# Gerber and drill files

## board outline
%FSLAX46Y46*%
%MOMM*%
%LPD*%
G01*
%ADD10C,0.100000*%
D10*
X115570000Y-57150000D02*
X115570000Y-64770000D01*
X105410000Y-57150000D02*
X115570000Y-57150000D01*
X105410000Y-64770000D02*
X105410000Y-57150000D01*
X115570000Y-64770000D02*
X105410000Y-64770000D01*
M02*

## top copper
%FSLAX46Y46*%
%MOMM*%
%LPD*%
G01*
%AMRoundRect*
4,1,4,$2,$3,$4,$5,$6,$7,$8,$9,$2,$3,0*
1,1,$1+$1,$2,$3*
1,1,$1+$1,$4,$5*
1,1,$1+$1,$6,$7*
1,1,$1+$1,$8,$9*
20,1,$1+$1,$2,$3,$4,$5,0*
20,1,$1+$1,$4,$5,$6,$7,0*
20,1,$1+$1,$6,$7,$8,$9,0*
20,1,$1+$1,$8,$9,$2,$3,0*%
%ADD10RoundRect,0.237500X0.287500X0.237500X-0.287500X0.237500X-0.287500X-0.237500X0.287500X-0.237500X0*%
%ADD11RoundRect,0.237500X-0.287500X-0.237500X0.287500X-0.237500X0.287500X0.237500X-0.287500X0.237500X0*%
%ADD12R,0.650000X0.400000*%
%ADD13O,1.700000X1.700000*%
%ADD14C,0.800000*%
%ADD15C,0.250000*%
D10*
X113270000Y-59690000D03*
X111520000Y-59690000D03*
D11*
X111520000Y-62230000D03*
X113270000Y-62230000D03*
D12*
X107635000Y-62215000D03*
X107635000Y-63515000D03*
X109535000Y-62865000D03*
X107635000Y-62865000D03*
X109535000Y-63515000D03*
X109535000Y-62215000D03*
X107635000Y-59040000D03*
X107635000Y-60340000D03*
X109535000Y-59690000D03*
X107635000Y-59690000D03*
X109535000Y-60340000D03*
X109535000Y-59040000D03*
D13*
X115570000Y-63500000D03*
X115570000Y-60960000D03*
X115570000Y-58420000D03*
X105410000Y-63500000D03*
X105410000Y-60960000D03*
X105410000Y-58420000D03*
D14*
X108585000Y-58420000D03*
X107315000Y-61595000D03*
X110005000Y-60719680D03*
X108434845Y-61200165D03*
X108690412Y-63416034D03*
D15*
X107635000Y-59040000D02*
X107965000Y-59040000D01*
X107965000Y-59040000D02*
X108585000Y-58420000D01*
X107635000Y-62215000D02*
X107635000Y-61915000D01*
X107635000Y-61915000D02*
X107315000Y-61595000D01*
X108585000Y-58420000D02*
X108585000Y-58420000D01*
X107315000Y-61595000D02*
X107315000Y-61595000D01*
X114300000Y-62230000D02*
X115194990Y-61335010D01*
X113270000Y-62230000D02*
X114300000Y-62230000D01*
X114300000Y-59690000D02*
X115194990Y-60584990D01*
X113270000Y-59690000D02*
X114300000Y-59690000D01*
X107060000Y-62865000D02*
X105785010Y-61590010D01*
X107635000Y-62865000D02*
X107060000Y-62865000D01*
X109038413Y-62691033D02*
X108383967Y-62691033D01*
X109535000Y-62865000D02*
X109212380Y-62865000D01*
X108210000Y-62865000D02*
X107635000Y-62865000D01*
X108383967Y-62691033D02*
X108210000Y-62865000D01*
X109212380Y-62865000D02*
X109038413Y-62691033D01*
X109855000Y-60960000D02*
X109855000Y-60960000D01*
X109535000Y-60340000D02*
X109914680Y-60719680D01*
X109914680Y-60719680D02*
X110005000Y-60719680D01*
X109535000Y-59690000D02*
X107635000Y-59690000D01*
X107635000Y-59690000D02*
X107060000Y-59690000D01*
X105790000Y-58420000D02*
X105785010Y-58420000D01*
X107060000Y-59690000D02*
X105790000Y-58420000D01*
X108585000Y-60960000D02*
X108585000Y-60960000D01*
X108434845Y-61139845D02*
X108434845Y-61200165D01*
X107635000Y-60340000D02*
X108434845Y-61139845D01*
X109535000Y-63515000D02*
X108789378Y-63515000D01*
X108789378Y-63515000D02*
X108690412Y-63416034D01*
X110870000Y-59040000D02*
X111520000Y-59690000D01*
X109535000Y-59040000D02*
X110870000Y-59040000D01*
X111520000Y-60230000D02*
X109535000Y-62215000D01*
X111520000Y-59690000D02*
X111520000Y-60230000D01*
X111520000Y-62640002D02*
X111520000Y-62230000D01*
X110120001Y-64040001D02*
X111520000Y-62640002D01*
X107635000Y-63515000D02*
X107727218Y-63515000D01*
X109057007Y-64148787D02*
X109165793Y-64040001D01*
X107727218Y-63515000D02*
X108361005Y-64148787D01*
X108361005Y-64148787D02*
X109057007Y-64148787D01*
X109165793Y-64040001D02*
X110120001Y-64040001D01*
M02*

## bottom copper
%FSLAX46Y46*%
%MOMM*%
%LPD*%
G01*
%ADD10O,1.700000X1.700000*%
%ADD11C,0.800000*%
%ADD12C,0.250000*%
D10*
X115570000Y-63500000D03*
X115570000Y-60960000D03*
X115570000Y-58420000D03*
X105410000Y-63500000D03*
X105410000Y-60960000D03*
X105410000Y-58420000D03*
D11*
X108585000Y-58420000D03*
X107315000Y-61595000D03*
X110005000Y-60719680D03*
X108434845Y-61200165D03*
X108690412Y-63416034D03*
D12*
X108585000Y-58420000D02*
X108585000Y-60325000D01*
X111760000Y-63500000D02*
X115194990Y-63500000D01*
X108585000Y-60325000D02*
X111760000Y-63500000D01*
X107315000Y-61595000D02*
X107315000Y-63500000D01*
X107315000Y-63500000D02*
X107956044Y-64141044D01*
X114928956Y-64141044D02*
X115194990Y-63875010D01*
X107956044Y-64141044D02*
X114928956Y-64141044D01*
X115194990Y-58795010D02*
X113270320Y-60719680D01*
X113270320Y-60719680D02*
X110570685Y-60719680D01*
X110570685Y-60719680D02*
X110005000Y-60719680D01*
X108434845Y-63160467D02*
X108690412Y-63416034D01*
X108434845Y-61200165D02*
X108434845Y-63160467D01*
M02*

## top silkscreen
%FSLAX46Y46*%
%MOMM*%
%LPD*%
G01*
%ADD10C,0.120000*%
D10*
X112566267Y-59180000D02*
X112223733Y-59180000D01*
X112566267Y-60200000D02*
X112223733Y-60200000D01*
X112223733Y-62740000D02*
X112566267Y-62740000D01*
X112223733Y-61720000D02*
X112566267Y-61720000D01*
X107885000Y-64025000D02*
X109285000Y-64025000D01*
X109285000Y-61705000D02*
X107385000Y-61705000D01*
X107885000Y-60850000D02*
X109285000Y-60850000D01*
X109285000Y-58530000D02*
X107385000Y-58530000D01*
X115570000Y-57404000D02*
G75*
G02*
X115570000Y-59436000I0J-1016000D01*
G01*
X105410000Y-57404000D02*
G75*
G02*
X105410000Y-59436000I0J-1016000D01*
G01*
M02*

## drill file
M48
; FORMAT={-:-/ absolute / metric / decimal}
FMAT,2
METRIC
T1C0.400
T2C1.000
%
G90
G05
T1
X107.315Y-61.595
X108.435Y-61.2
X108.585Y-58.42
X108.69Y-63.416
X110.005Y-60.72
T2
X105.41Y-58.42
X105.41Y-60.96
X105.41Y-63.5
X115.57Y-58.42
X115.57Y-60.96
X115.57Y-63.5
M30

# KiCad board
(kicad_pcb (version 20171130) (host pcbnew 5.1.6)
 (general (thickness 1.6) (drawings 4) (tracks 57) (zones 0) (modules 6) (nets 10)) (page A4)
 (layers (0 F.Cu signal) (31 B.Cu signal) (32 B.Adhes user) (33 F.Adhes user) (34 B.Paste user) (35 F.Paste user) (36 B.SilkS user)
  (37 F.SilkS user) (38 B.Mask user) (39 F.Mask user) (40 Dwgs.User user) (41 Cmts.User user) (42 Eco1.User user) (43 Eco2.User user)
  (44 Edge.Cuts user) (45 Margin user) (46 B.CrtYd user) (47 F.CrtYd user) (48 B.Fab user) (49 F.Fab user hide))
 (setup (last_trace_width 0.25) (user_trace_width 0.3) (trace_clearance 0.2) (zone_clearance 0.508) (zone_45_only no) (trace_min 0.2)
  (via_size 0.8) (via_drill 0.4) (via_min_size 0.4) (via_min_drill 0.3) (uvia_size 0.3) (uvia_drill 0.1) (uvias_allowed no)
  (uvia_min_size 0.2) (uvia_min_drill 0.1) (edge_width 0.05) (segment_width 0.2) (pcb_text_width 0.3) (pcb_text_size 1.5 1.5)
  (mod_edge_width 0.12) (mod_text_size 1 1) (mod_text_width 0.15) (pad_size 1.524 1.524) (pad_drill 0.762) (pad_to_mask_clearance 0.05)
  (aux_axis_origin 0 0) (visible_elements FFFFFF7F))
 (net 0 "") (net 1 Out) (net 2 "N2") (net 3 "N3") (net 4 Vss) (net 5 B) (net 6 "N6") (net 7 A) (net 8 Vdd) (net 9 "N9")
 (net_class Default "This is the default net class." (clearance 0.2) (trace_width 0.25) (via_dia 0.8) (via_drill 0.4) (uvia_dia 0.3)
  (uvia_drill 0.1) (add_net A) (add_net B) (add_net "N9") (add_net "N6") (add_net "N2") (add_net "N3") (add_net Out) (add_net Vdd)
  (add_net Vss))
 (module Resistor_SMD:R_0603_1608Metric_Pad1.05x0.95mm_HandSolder (layer F.Cu) (at 112.395 59.69 180)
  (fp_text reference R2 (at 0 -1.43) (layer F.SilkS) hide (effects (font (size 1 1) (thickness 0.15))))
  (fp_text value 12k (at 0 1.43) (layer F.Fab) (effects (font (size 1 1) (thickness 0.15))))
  (fp_line (start -0.171267 0.51) (end 0.171267 0.51) (layer F.SilkS) (width 0.12))
  (fp_line (start -0.171267 -0.51) (end 0.171267 -0.51) (layer F.SilkS) (width 0.12))
  (pad 1 smd roundrect (at -0.875 0 180) (size 1.05 0.95) (layers F.Cu F.Paste F.Mask) (roundrect_rratio 0.25) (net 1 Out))
  (pad 2 smd roundrect (at 0.875 0 180) (size 1.05 0.95) (layers F.Cu F.Paste F.Mask) (roundrect_rratio 0.25) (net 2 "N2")))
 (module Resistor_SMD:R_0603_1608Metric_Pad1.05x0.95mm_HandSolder (layer F.Cu) (at 112.395 62.23)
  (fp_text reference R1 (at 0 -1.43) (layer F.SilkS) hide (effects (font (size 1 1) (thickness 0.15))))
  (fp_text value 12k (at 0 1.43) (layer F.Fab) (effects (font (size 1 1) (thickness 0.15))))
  (fp_line (start -0.171267 0.51) (end 0.171267 0.51) (layer F.SilkS) (width 0.12))
  (fp_line (start -0.171267 -0.51) (end 0.171267 -0.51) (layer F.SilkS) (width 0.12))
  (pad 1 smd roundrect (at -0.875 0) (size 1.05 0.95) (layers F.Cu F.Paste F.Mask) (roundrect_rratio 0.25) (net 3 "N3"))
  (pad 2 smd roundrect (at 0.875 0) (size 1.05 0.95) (layers F.Cu F.Paste F.Mask) (roundrect_rratio 0.25) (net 1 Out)))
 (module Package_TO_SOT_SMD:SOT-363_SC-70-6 (layer F.Cu) (at 108.585 62.865)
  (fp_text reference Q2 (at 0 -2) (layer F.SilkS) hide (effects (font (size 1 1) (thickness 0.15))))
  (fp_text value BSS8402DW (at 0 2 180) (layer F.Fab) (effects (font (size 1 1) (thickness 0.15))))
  (fp_line (start -0.7 1.16) (end 0.7 1.16) (layer F.SilkS) (width 0.12))
  (fp_line (start 0.7 -1.16) (end -1.2 -1.16) (layer F.SilkS) (width 0.12))
  (pad 1 smd rect (at -0.95 -0.65) (size 0.65 0.4) (layers F.Cu F.Paste F.Mask) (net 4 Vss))
  (pad 3 smd rect (at -0.95 0.65) (size 0.65 0.4) (layers F.Cu F.Paste F.Mask) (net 3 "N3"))
  (pad 5 smd rect (at 0.95 0) (size 0.65 0.4) (layers F.Cu F.Paste F.Mask) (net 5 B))
  (pad 2 smd rect (at -0.95 0) (size 0.65 0.4) (layers F.Cu F.Paste F.Mask) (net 5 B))
  (pad 4 smd rect (at 0.95 0.65) (size 0.65 0.4) (layers F.Cu F.Paste F.Mask) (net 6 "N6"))
  (pad 6 smd rect (at 0.95 -0.65) (size 0.65 0.4) (layers F.Cu F.Paste F.Mask) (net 2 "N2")))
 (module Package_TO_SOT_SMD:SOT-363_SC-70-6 (layer F.Cu) (at 108.585 59.69)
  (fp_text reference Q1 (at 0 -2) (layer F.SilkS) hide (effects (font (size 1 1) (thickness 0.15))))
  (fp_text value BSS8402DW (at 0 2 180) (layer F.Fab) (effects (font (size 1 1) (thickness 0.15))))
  (fp_line (start -0.7 1.16) (end 0.7 1.16) (layer F.SilkS) (width 0.12))
  (fp_line (start 0.7 -1.16) (end -1.2 -1.16) (layer F.SilkS) (width 0.12))
  (pad 1 smd rect (at -0.95 -0.65) (size 0.65 0.4) (layers F.Cu F.Paste F.Mask) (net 4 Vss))
  (pad 3 smd rect (at -0.95 0.65) (size 0.65 0.4) (layers F.Cu F.Paste F.Mask) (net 6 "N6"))
  (pad 5 smd rect (at 0.95 0) (size 0.65 0.4) (layers F.Cu F.Paste F.Mask) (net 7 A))
  (pad 2 smd rect (at -0.95 0) (size 0.65 0.4) (layers F.Cu F.Paste F.Mask) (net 7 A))
  (pad 4 smd rect (at 0.95 0.65) (size 0.65 0.4) (layers F.Cu F.Paste F.Mask) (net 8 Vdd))
  (pad 6 smd rect (at 0.95 -0.65) (size 0.65 0.4) (layers F.Cu F.Paste F.Mask) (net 2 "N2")))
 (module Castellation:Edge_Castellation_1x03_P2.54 (layer F.Cu) (at 115.57 58.42)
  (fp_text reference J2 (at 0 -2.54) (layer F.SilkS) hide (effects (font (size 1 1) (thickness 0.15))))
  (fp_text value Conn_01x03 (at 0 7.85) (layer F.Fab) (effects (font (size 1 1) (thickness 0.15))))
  (fp_arc (start 0 0) (end 0 1.016) (angle -180) (layer F.SilkS) (width 0.12))
  (pad 3 thru_hole oval (at 0 5.08) (size 1.7 1.7) (drill 1) (layers *.Cu *.Mask) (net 4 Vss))
  (pad 2 thru_hole oval (at 0 2.54) (size 1.7 1.7) (drill 1) (layers *.Cu *.Mask) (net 1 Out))
  (pad 1 thru_hole oval (at 0 0) (size 1.7 1.7) (drill 1) (layers *.Cu *.Mask) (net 8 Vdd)))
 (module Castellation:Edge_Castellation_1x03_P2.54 (layer F.Cu) (at 105.41 58.42)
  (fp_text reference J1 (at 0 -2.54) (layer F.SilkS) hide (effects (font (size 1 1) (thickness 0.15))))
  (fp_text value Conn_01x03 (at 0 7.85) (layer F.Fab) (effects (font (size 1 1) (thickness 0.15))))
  (fp_arc (start 0 0) (end 0 1.016) (angle -180) (layer F.SilkS) (width 0.12))
  (pad 3 thru_hole oval (at 0 5.08) (size 1.7 1.7) (drill 1) (layers *.Cu *.Mask) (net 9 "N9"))
  (pad 2 thru_hole oval (at 0 2.54) (size 1.7 1.7) (drill 1) (layers *.Cu *.Mask) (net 5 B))
  (pad 1 thru_hole oval (at 0 0) (size 1.7 1.7) (drill 1) (layers *.Cu *.Mask) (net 7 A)))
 (gr_line (start 115.57 57.15) (end 115.57 64.77) (layer Edge.Cuts) (width 0.1))
 (gr_line (start 105.41 57.15) (end 115.57 57.15) (layer Edge.Cuts) (width 0.1))
 (gr_line (start 105.41 64.77) (end 105.41 57.15) (layer Edge.Cuts) (width 0.1))
 (gr_line (start 115.57 64.77) (end 105.41 64.77) (layer Edge.Cuts) (width 0.1))
 (segment (start 107.635 59.04) (end 107.965 59.04) (width 0.25) (layer F.Cu) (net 4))
 (segment (start 107.965 59.04) (end 108.585 58.42) (width 0.25) (layer F.Cu) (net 4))
 (segment (start 107.635 62.215) (end 107.635 61.915) (width 0.25) (layer F.Cu) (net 4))
 (segment (start 107.635 61.915) (end 107.315 61.595) (width 0.25) (layer F.Cu) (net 4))
 (segment (start 108.585 58.42) (end 108.585 58.42) (width 0.25) (layer F.Cu) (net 4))
 (via (at 108.585 58.42) (size 0.8) (drill 0.4) (layers F.Cu B.Cu) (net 4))
 (segment (start 107.315 61.595) (end 107.315 61.595) (width 0.25) (layer F.Cu) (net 4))
 (via (at 107.315 61.595) (size 0.8) (drill 0.4) (layers F.Cu B.Cu) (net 4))
 (segment (start 108.585 58.42) (end 108.585 60.325) (width 0.25) (layer B.Cu) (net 4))
 (segment (start 111.76 63.5) (end 115.19499 63.5) (width 0.25) (layer B.Cu) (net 4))
 (segment (start 108.585 60.325) (end 111.76 63.5) (width 0.25) (layer B.Cu) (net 4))
 (segment (start 107.315 61.595) (end 107.315 63.5) (width 0.25) (layer B.Cu) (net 4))
 (segment (start 107.315 63.5) (end 107.956044 64.141044) (width 0.25) (layer B.Cu) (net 4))
 (segment (start 114.928956 64.141044) (end 115.19499 63.87501) (width 0.25) (layer B.Cu) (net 4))
 (segment (start 107.956044 64.141044) (end 114.928956 64.141044) (width 0.25) (layer B.Cu) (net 4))
 (segment (start 114.3 62.23) (end 115.19499 61.33501) (width 0.25) (layer F.Cu) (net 1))
 (segment (start 113.27 62.23) (end 114.3 62.23) (width 0.25) (layer F.Cu) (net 1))
 (segment (start 114.3 59.69) (end 115.19499 60.58499) (width 0.25) (layer F.Cu) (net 1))
 (segment (start 113.27 59.69) (end 114.3 59.69) (width 0.25) (layer F.Cu) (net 1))
 (segment (start 107.06 62.865) (end 105.78501 61.59001) (width 0.25) (layer F.Cu) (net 5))
 (segment (start 107.635 62.865) (end 107.06 62.865) (width 0.25) (layer F.Cu) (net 5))
 (segment (start 109.038413 62.691033) (end 108.383967 62.691033) (width 0.25) (layer F.Cu) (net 5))
 (segment (start 109.535 62.865) (end 109.21238 62.865) (width 0.25) (layer F.Cu) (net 5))
 (segment (start 108.21 62.865) (end 107.635 62.865) (width 0.25) (layer F.Cu) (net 5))
 (segment (start 108.383967 62.691033) (end 108.21 62.865) (width 0.25) (layer F.Cu) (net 5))
 (segment (start 109.21238 62.865) (end 109.038413 62.691033) (width 0.25) (layer F.Cu) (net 5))
 (segment (start 109.855 60.96) (end 109.855 60.96) (width 0.25) (layer F.Cu) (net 8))
 (via (at 110.005 60.71968) (size 0.8) (drill 0.4) (layers F.Cu B.Cu) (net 8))
 (segment (start 109.535 60.34) (end 109.91468 60.71968) (width 0.25) (layer F.Cu) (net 8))
 (segment (start 115.19499 58.79501) (end 113.27032 60.71968) (width 0.25) (layer B.Cu) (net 8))
 (segment (start 113.27032 60.71968) (end 110.570685 60.71968) (width 0.25) (layer B.Cu) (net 8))
 (segment (start 110.570685 60.71968) (end 110.005 60.71968) (width 0.25) (layer B.Cu) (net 8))
 (segment (start 109.91468 60.71968) (end 110.005 60.71968) (width 0.25) (layer F.Cu) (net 8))
 (segment (start 109.535 59.69) (end 107.635 59.69) (width 0.25) (layer F.Cu) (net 7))
 (segment (start 107.635 59.69) (end 107.06 59.69) (width 0.25) (layer F.Cu) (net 7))
 (segment (start 105.79 58.42) (end 105.78501 58.42) (width 0.25) (layer F.Cu) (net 7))
 (segment (start 107.06 59.69) (end 105.79 58.42) (width 0.25) (layer F.Cu) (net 7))
 (segment (start 108.585 60.96) (end 108.585 60.96) (width 0.25) (layer F.Cu) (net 6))
 (via (at 108.434845 61.200165) (size 0.8) (drill 0.4) (layers F.Cu B.Cu) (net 6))
 (segment (start 108.434845 61.139845) (end 108.434845 61.200165) (width 0.25) (layer F.Cu) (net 6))
 (segment (start 107.635 60.34) (end 108.434845 61.139845) (width 0.25) (layer F.Cu) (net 6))
 (segment (start 108.434845 63.160467) (end 108.690412 63.416034) (width 0.25) (layer B.Cu) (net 6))
 (segment (start 108.434845 61.200165) (end 108.434845 63.160467) (width 0.25) (layer B.Cu) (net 6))
 (segment (start 109.535 63.515) (end 108.789378 63.515) (width 0.25) (layer F.Cu) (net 6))
 (segment (start 108.789378 63.515) (end 108.690412 63.416034) (width 0.25) (layer F.Cu) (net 6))
 (via (at 108.690412 63.416034) (size 0.8) (drill 0.4) (layers F.Cu B.Cu) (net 6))
 (segment (start 110.87 59.04) (end 111.52 59.69) (width 0.25) (layer F.Cu) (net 2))
 (segment (start 109.535 59.04) (end 110.87 59.04) (width 0.25) (layer F.Cu) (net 2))
 (segment (start 111.52 60.23) (end 109.535 62.215) (width 0.25) (layer F.Cu) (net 2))
 (segment (start 111.52 59.69) (end 111.52 60.23) (width 0.25) (layer F.Cu) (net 2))
 (segment (start 111.52 62.640002) (end 111.52 62.23) (width 0.25) (layer F.Cu) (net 3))
 (segment (start 110.120001 64.040001) (end 111.52 62.640002) (width 0.25) (layer F.Cu) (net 3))
 (segment (start 107.635 63.515) (end 107.727218 63.515) (width 0.25) (layer F.Cu) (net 3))
 (segment (start 109.057007 64.148787) (end 109.165793 64.040001) (width 0.25) (layer F.Cu) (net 3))
 (segment (start 107.727218 63.515) (end 108.361005 64.148787) (width 0.25) (layer F.Cu) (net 3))
 (segment (start 108.361005 64.148787) (end 109.057007 64.148787) (width 0.25) (layer F.Cu) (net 3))
 (segment (start 109.165793 64.040001) (end 110.120001 64.040001) (width 0.25) (layer F.Cu) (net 3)))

